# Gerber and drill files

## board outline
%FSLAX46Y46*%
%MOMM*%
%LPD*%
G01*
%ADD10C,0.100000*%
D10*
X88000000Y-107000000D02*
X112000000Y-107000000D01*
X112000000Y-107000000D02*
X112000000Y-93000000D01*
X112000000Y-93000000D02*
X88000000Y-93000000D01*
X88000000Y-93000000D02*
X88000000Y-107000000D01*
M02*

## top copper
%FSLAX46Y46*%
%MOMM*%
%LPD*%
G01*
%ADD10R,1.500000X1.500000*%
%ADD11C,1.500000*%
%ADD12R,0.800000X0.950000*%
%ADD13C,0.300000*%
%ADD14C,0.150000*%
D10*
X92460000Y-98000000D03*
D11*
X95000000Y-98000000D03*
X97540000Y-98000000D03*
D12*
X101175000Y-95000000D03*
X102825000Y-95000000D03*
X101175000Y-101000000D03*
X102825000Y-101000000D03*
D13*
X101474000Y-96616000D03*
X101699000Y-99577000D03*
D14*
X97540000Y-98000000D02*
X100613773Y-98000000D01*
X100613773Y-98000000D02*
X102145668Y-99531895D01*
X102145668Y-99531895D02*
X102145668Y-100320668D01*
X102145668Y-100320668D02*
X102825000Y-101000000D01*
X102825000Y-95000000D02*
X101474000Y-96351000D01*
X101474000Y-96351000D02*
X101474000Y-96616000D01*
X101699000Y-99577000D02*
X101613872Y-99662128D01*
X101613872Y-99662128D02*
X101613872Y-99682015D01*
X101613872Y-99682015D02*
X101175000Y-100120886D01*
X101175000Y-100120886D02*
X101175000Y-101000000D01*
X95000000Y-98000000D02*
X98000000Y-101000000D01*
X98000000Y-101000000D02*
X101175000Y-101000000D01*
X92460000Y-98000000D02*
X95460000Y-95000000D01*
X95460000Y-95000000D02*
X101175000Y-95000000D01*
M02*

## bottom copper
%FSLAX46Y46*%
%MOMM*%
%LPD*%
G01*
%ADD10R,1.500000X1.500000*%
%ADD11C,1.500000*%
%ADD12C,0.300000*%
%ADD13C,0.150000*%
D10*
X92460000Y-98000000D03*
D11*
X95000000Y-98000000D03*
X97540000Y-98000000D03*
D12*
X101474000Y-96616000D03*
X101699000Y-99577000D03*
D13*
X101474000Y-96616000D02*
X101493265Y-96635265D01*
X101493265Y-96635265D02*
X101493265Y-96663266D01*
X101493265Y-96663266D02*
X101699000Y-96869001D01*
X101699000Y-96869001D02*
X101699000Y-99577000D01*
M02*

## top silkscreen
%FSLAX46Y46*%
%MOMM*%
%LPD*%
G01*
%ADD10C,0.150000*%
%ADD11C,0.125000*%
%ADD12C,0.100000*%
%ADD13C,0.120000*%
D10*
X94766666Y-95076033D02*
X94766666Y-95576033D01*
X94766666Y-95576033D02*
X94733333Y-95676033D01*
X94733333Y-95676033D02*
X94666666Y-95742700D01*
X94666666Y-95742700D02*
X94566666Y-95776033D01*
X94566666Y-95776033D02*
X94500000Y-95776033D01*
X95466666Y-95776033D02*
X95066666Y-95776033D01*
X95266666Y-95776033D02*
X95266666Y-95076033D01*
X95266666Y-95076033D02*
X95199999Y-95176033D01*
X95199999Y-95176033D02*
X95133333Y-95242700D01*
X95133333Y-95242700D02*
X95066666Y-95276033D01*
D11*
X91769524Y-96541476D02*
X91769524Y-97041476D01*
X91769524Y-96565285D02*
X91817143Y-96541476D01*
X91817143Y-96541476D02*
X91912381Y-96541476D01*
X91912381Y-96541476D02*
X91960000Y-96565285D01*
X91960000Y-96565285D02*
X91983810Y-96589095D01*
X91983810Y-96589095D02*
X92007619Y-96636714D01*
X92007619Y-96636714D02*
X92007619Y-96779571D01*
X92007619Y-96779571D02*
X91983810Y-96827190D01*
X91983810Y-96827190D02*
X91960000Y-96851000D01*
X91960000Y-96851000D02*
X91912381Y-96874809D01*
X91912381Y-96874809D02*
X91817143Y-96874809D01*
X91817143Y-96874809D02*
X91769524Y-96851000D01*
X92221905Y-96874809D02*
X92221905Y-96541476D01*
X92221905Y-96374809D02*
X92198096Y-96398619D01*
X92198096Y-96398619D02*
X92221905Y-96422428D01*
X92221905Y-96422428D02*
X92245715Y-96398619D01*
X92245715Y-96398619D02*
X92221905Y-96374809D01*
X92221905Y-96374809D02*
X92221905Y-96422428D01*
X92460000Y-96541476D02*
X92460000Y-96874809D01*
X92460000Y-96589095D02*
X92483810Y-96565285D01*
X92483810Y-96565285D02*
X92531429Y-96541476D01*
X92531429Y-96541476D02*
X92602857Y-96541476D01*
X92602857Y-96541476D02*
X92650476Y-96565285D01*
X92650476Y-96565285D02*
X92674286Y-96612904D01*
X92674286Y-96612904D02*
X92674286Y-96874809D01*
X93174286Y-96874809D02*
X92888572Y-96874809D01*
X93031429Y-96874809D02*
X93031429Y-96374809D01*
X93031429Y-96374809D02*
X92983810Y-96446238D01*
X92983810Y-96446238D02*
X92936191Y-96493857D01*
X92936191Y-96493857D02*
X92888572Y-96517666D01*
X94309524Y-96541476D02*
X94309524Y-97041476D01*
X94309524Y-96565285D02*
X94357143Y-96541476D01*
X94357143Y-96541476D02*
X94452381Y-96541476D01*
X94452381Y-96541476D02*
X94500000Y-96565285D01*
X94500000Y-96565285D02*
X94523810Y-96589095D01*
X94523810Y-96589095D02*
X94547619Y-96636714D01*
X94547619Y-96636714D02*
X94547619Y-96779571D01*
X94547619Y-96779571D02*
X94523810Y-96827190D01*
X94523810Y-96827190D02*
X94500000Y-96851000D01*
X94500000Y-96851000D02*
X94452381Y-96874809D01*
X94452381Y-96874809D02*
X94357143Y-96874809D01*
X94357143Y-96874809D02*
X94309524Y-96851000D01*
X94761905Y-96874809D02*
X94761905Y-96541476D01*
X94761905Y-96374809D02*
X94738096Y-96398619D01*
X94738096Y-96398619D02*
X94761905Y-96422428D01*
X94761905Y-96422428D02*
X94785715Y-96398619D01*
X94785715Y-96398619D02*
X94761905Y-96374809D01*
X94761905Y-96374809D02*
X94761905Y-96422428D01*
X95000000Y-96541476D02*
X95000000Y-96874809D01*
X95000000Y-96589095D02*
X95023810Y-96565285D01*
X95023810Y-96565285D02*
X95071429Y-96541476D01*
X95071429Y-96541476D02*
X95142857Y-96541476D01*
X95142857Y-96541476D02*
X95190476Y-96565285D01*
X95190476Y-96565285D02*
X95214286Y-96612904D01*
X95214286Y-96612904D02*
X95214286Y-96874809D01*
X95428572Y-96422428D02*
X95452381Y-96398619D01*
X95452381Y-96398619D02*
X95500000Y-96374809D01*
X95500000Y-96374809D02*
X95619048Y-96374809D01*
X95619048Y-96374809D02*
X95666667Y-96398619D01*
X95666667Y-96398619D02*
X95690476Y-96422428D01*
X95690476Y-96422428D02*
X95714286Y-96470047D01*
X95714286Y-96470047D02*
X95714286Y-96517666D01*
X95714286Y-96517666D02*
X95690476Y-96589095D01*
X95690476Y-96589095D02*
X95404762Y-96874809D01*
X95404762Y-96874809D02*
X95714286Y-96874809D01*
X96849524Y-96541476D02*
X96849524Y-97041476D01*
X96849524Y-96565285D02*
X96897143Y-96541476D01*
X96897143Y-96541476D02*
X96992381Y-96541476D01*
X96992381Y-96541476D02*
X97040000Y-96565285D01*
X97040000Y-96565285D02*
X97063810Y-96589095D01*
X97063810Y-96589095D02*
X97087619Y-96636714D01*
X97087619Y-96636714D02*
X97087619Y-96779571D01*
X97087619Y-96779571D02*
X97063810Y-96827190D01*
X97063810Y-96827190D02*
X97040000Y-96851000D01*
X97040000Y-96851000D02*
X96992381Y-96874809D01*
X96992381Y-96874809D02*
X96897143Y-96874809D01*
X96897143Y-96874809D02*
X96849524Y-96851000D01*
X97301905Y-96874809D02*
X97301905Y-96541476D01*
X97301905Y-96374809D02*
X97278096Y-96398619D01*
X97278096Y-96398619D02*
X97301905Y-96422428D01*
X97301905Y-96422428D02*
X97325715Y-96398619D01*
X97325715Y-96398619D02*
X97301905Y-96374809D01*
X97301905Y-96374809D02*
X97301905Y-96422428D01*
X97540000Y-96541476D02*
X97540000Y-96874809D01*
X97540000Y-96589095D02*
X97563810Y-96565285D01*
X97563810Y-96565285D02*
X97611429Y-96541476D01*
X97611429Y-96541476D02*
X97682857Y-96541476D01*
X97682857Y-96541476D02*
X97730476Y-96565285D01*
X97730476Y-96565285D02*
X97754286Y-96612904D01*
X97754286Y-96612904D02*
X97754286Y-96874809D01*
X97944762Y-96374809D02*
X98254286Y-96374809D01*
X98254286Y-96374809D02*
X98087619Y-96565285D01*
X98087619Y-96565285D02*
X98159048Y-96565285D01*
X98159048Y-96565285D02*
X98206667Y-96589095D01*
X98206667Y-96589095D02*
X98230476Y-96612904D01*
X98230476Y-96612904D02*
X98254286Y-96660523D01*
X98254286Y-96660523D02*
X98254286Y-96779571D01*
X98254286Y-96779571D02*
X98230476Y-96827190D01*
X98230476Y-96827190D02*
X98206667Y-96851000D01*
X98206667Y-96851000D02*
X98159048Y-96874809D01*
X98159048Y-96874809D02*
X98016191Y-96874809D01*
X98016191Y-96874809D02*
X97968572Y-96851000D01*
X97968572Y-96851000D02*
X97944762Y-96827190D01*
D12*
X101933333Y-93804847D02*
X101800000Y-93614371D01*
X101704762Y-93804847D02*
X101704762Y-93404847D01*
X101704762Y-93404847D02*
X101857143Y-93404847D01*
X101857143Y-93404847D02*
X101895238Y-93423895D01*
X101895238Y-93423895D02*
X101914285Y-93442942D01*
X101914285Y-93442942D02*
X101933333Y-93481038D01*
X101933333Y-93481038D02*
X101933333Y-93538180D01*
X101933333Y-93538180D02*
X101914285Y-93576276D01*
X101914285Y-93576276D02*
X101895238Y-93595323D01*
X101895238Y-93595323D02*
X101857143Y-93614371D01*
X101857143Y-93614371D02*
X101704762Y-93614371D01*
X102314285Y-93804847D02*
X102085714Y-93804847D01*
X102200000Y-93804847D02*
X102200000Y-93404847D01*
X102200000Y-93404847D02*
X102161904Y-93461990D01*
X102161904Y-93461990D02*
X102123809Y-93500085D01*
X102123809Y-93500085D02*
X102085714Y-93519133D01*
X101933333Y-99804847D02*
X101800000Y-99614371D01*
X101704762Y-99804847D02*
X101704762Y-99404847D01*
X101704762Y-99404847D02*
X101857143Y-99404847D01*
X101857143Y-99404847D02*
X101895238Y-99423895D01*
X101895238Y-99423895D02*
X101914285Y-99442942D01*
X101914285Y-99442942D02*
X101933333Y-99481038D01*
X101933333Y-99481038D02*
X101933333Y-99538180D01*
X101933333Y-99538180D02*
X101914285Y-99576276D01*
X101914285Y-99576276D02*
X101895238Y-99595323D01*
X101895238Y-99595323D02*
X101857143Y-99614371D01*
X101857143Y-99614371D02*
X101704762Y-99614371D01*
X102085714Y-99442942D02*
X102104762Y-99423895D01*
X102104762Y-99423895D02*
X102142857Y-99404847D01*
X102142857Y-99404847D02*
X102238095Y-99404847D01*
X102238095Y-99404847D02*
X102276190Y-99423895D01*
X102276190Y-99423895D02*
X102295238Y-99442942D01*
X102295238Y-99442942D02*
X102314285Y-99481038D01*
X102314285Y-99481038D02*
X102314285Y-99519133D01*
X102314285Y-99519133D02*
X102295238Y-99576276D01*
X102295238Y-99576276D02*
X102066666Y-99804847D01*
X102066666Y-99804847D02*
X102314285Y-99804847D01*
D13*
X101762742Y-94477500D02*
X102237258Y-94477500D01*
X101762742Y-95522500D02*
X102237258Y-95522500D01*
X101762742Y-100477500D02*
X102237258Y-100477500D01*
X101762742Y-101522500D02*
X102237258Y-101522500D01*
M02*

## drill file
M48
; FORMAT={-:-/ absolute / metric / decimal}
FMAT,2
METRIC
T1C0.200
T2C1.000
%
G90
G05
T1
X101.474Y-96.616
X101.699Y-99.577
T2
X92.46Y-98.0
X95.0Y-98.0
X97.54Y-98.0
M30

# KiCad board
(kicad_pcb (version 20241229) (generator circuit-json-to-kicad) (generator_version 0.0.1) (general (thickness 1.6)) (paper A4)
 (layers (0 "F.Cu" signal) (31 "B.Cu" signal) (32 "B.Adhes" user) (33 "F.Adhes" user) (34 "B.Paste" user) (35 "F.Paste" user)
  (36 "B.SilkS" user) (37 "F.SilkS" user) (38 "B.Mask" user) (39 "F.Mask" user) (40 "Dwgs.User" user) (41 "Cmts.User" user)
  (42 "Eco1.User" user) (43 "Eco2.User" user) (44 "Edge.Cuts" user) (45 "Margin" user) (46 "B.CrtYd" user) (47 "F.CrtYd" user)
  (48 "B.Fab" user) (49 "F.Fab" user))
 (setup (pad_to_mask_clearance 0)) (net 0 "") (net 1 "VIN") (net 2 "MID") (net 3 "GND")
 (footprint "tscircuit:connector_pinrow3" (layer F.Cu) (at 95 98 0)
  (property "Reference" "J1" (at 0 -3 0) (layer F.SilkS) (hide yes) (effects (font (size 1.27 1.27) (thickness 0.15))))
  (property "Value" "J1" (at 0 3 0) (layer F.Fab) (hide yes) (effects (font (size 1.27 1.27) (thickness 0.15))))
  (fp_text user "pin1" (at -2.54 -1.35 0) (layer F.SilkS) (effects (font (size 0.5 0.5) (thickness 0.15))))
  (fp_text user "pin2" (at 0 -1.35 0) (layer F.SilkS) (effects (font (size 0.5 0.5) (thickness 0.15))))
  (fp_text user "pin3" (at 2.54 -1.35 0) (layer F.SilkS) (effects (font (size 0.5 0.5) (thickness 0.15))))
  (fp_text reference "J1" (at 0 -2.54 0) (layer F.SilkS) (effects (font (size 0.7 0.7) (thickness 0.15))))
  (pad "1" thru_hole rect (at -2.54 0 0) (size 1.5 1.5) (drill 1) (layers *.Cu *.Mask) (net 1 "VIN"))
  (pad "2" thru_hole circle (at 0 0 0) (size 1.5 1.5) (drill 1) (layers *.Cu *.Mask) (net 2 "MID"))
  (pad "3" thru_hole circle (at 2.54 0 0) (size 1.5 1.5) (drill 1) (layers *.Cu *.Mask) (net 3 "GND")))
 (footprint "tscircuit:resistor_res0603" (layer F.Cu) (at 102 95 0)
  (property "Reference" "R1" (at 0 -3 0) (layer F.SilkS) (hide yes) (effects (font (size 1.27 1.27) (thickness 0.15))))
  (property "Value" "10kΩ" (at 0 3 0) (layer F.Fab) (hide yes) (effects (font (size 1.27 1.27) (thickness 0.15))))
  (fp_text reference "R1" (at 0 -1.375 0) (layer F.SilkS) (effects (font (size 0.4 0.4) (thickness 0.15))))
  (fp_line (start -0.23725799999999997 -0.5225) (end 0.2372580000000002 -0.5225) (stroke (width 0.12) (type default)) (layer F.SilkS))
  (fp_line (start -0.23725799999999997 0.5225) (end 0.2372580000000002 0.5225) (stroke (width 0.12) (type default)) (layer F.SilkS))
  (pad "1" smd rect (at -0.825 0 0) (size 0.8 0.95) (layers F.Cu F.Mask) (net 1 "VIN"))
  (pad "2" smd rect (at 0.8250000000000002 0 0) (size 0.8 0.95) (layers F.Cu F.Mask) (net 2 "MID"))
  (pad "" smd rect (at -0.825 0 0) (size 0.5599999999999999 0.6649999999999999) (layers F.Paste))
  (pad "" smd rect (at 0.8250000000000002 0 0) (size 0.5599999999999999 0.6649999999999999) (layers F.Paste)))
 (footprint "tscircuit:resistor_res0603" (layer F.Cu) (at 102 101 0)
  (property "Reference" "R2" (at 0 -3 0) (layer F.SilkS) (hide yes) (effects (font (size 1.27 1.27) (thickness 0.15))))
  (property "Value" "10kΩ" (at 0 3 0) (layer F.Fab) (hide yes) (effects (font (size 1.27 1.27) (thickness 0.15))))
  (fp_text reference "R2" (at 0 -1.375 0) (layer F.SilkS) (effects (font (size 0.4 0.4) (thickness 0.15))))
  (fp_line (start -0.23725799999999997 -0.5225) (end 0.2372580000000002 -0.5225) (stroke (width 0.12) (type default)) (layer F.SilkS))
  (fp_line (start -0.23725799999999997 0.5225) (end 0.2372580000000002 0.5225) (stroke (width 0.12) (type default)) (layer F.SilkS))
  (pad "1" smd rect (at -0.825 0 0) (size 0.8 0.95) (layers F.Cu F.Mask) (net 2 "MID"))
  (pad "2" smd rect (at 0.8250000000000002 0 0) (size 0.8 0.95) (layers F.Cu F.Mask) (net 3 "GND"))
  (pad "" smd rect (at -0.825 0 0) (size 0.5599999999999999 0.6649999999999999) (layers F.Paste))
  (pad "" smd rect (at 0.8250000000000002 0 0) (size 0.5599999999999999 0.6649999999999999) (layers F.Paste)))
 (segment (start 97.54 98) (end 100.61377303374535 98) (width 0.15) (layer F.Cu) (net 3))
 (segment (start 100.61377303374535 98) (end 102.14566818909657 99.53189515535122) (width 0.15) (layer F.Cu) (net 3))
 (segment (start 102.14566818909657 99.53189515535122) (end 102.14566818909657 100.32066818909657) (width 0.15) (layer F.Cu) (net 3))
 (segment (start 102.14566818909657 100.32066818909657) (end 102.825 101) (width 0.15) (layer F.Cu) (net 3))
 (segment (start 102.825 95) (end 101.474 96.351) (width 0.15) (layer F.Cu) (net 2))
 (segment (start 101.474 96.351) (end 101.474 96.616) (width 0.15) (layer F.Cu) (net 2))
 (segment (start 101.474 96.616) (end 101.4932646028625 96.6352646028625) (width 0.15) (layer B.Cu) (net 2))
 (segment (start 101.4932646028625 96.6352646028625) (end 101.4932646028625 96.66326571586013) (width 0.15) (layer B.Cu) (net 2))
 (segment (start 101.4932646028625 96.66326571586013) (end 101.699 96.86900111299764) (width 0.15) (layer B.Cu) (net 2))
 (segment (start 101.699 96.86900111299764) (end 101.699 99.577) (width 0.15) (layer B.Cu) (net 2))
 (segment (start 101.699 99.577) (end 101.61387153996071 99.66212846003928) (width 0.15) (layer F.Cu) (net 2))
 (segment (start 101.61387153996071 99.66212846003928) (end 101.61387153996071 99.68201458898672) (width 0.15) (layer F.Cu) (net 2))
 (segment (start 101.61387153996071 99.68201458898672) (end 101.175 100.12088612894743) (width 0.15) (layer F.Cu) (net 2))
 (segment (start 101.175 100.12088612894743) (end 101.175 101) (width 0.15) (layer F.Cu) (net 2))
 (segment (start 95 98) (end 98 101) (width 0.15) (layer F.Cu) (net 2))
 (segment (start 98 101) (end 101.175 101) (width 0.15) (layer F.Cu) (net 2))
 (segment (start 92.46 98) (end 95.46 95) (width 0.15) (layer F.Cu) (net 1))
 (segment (start 95.46 95) (end 101.175 95) (width 0.15) (layer F.Cu) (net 1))
 (gr_line (start 88 107) (end 112 107) (width 0.1) (layer Edge.Cuts))
 (gr_line (start 112 107) (end 112 93) (width 0.1) (layer Edge.Cuts))
 (gr_line (start 112 93) (end 88 93) (width 0.1) (layer Edge.Cuts))
 (gr_line (start 88 93) (end 88 107) (width 0.1) (layer Edge.Cuts))
 (via (at 101.474 96.616) (size 0.3) (drill 0.2) (layers F.Cu B.Cu) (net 2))
 (via (at 101.699 99.577) (size 0.3) (drill 0.2) (layers F.Cu B.Cu) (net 2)))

